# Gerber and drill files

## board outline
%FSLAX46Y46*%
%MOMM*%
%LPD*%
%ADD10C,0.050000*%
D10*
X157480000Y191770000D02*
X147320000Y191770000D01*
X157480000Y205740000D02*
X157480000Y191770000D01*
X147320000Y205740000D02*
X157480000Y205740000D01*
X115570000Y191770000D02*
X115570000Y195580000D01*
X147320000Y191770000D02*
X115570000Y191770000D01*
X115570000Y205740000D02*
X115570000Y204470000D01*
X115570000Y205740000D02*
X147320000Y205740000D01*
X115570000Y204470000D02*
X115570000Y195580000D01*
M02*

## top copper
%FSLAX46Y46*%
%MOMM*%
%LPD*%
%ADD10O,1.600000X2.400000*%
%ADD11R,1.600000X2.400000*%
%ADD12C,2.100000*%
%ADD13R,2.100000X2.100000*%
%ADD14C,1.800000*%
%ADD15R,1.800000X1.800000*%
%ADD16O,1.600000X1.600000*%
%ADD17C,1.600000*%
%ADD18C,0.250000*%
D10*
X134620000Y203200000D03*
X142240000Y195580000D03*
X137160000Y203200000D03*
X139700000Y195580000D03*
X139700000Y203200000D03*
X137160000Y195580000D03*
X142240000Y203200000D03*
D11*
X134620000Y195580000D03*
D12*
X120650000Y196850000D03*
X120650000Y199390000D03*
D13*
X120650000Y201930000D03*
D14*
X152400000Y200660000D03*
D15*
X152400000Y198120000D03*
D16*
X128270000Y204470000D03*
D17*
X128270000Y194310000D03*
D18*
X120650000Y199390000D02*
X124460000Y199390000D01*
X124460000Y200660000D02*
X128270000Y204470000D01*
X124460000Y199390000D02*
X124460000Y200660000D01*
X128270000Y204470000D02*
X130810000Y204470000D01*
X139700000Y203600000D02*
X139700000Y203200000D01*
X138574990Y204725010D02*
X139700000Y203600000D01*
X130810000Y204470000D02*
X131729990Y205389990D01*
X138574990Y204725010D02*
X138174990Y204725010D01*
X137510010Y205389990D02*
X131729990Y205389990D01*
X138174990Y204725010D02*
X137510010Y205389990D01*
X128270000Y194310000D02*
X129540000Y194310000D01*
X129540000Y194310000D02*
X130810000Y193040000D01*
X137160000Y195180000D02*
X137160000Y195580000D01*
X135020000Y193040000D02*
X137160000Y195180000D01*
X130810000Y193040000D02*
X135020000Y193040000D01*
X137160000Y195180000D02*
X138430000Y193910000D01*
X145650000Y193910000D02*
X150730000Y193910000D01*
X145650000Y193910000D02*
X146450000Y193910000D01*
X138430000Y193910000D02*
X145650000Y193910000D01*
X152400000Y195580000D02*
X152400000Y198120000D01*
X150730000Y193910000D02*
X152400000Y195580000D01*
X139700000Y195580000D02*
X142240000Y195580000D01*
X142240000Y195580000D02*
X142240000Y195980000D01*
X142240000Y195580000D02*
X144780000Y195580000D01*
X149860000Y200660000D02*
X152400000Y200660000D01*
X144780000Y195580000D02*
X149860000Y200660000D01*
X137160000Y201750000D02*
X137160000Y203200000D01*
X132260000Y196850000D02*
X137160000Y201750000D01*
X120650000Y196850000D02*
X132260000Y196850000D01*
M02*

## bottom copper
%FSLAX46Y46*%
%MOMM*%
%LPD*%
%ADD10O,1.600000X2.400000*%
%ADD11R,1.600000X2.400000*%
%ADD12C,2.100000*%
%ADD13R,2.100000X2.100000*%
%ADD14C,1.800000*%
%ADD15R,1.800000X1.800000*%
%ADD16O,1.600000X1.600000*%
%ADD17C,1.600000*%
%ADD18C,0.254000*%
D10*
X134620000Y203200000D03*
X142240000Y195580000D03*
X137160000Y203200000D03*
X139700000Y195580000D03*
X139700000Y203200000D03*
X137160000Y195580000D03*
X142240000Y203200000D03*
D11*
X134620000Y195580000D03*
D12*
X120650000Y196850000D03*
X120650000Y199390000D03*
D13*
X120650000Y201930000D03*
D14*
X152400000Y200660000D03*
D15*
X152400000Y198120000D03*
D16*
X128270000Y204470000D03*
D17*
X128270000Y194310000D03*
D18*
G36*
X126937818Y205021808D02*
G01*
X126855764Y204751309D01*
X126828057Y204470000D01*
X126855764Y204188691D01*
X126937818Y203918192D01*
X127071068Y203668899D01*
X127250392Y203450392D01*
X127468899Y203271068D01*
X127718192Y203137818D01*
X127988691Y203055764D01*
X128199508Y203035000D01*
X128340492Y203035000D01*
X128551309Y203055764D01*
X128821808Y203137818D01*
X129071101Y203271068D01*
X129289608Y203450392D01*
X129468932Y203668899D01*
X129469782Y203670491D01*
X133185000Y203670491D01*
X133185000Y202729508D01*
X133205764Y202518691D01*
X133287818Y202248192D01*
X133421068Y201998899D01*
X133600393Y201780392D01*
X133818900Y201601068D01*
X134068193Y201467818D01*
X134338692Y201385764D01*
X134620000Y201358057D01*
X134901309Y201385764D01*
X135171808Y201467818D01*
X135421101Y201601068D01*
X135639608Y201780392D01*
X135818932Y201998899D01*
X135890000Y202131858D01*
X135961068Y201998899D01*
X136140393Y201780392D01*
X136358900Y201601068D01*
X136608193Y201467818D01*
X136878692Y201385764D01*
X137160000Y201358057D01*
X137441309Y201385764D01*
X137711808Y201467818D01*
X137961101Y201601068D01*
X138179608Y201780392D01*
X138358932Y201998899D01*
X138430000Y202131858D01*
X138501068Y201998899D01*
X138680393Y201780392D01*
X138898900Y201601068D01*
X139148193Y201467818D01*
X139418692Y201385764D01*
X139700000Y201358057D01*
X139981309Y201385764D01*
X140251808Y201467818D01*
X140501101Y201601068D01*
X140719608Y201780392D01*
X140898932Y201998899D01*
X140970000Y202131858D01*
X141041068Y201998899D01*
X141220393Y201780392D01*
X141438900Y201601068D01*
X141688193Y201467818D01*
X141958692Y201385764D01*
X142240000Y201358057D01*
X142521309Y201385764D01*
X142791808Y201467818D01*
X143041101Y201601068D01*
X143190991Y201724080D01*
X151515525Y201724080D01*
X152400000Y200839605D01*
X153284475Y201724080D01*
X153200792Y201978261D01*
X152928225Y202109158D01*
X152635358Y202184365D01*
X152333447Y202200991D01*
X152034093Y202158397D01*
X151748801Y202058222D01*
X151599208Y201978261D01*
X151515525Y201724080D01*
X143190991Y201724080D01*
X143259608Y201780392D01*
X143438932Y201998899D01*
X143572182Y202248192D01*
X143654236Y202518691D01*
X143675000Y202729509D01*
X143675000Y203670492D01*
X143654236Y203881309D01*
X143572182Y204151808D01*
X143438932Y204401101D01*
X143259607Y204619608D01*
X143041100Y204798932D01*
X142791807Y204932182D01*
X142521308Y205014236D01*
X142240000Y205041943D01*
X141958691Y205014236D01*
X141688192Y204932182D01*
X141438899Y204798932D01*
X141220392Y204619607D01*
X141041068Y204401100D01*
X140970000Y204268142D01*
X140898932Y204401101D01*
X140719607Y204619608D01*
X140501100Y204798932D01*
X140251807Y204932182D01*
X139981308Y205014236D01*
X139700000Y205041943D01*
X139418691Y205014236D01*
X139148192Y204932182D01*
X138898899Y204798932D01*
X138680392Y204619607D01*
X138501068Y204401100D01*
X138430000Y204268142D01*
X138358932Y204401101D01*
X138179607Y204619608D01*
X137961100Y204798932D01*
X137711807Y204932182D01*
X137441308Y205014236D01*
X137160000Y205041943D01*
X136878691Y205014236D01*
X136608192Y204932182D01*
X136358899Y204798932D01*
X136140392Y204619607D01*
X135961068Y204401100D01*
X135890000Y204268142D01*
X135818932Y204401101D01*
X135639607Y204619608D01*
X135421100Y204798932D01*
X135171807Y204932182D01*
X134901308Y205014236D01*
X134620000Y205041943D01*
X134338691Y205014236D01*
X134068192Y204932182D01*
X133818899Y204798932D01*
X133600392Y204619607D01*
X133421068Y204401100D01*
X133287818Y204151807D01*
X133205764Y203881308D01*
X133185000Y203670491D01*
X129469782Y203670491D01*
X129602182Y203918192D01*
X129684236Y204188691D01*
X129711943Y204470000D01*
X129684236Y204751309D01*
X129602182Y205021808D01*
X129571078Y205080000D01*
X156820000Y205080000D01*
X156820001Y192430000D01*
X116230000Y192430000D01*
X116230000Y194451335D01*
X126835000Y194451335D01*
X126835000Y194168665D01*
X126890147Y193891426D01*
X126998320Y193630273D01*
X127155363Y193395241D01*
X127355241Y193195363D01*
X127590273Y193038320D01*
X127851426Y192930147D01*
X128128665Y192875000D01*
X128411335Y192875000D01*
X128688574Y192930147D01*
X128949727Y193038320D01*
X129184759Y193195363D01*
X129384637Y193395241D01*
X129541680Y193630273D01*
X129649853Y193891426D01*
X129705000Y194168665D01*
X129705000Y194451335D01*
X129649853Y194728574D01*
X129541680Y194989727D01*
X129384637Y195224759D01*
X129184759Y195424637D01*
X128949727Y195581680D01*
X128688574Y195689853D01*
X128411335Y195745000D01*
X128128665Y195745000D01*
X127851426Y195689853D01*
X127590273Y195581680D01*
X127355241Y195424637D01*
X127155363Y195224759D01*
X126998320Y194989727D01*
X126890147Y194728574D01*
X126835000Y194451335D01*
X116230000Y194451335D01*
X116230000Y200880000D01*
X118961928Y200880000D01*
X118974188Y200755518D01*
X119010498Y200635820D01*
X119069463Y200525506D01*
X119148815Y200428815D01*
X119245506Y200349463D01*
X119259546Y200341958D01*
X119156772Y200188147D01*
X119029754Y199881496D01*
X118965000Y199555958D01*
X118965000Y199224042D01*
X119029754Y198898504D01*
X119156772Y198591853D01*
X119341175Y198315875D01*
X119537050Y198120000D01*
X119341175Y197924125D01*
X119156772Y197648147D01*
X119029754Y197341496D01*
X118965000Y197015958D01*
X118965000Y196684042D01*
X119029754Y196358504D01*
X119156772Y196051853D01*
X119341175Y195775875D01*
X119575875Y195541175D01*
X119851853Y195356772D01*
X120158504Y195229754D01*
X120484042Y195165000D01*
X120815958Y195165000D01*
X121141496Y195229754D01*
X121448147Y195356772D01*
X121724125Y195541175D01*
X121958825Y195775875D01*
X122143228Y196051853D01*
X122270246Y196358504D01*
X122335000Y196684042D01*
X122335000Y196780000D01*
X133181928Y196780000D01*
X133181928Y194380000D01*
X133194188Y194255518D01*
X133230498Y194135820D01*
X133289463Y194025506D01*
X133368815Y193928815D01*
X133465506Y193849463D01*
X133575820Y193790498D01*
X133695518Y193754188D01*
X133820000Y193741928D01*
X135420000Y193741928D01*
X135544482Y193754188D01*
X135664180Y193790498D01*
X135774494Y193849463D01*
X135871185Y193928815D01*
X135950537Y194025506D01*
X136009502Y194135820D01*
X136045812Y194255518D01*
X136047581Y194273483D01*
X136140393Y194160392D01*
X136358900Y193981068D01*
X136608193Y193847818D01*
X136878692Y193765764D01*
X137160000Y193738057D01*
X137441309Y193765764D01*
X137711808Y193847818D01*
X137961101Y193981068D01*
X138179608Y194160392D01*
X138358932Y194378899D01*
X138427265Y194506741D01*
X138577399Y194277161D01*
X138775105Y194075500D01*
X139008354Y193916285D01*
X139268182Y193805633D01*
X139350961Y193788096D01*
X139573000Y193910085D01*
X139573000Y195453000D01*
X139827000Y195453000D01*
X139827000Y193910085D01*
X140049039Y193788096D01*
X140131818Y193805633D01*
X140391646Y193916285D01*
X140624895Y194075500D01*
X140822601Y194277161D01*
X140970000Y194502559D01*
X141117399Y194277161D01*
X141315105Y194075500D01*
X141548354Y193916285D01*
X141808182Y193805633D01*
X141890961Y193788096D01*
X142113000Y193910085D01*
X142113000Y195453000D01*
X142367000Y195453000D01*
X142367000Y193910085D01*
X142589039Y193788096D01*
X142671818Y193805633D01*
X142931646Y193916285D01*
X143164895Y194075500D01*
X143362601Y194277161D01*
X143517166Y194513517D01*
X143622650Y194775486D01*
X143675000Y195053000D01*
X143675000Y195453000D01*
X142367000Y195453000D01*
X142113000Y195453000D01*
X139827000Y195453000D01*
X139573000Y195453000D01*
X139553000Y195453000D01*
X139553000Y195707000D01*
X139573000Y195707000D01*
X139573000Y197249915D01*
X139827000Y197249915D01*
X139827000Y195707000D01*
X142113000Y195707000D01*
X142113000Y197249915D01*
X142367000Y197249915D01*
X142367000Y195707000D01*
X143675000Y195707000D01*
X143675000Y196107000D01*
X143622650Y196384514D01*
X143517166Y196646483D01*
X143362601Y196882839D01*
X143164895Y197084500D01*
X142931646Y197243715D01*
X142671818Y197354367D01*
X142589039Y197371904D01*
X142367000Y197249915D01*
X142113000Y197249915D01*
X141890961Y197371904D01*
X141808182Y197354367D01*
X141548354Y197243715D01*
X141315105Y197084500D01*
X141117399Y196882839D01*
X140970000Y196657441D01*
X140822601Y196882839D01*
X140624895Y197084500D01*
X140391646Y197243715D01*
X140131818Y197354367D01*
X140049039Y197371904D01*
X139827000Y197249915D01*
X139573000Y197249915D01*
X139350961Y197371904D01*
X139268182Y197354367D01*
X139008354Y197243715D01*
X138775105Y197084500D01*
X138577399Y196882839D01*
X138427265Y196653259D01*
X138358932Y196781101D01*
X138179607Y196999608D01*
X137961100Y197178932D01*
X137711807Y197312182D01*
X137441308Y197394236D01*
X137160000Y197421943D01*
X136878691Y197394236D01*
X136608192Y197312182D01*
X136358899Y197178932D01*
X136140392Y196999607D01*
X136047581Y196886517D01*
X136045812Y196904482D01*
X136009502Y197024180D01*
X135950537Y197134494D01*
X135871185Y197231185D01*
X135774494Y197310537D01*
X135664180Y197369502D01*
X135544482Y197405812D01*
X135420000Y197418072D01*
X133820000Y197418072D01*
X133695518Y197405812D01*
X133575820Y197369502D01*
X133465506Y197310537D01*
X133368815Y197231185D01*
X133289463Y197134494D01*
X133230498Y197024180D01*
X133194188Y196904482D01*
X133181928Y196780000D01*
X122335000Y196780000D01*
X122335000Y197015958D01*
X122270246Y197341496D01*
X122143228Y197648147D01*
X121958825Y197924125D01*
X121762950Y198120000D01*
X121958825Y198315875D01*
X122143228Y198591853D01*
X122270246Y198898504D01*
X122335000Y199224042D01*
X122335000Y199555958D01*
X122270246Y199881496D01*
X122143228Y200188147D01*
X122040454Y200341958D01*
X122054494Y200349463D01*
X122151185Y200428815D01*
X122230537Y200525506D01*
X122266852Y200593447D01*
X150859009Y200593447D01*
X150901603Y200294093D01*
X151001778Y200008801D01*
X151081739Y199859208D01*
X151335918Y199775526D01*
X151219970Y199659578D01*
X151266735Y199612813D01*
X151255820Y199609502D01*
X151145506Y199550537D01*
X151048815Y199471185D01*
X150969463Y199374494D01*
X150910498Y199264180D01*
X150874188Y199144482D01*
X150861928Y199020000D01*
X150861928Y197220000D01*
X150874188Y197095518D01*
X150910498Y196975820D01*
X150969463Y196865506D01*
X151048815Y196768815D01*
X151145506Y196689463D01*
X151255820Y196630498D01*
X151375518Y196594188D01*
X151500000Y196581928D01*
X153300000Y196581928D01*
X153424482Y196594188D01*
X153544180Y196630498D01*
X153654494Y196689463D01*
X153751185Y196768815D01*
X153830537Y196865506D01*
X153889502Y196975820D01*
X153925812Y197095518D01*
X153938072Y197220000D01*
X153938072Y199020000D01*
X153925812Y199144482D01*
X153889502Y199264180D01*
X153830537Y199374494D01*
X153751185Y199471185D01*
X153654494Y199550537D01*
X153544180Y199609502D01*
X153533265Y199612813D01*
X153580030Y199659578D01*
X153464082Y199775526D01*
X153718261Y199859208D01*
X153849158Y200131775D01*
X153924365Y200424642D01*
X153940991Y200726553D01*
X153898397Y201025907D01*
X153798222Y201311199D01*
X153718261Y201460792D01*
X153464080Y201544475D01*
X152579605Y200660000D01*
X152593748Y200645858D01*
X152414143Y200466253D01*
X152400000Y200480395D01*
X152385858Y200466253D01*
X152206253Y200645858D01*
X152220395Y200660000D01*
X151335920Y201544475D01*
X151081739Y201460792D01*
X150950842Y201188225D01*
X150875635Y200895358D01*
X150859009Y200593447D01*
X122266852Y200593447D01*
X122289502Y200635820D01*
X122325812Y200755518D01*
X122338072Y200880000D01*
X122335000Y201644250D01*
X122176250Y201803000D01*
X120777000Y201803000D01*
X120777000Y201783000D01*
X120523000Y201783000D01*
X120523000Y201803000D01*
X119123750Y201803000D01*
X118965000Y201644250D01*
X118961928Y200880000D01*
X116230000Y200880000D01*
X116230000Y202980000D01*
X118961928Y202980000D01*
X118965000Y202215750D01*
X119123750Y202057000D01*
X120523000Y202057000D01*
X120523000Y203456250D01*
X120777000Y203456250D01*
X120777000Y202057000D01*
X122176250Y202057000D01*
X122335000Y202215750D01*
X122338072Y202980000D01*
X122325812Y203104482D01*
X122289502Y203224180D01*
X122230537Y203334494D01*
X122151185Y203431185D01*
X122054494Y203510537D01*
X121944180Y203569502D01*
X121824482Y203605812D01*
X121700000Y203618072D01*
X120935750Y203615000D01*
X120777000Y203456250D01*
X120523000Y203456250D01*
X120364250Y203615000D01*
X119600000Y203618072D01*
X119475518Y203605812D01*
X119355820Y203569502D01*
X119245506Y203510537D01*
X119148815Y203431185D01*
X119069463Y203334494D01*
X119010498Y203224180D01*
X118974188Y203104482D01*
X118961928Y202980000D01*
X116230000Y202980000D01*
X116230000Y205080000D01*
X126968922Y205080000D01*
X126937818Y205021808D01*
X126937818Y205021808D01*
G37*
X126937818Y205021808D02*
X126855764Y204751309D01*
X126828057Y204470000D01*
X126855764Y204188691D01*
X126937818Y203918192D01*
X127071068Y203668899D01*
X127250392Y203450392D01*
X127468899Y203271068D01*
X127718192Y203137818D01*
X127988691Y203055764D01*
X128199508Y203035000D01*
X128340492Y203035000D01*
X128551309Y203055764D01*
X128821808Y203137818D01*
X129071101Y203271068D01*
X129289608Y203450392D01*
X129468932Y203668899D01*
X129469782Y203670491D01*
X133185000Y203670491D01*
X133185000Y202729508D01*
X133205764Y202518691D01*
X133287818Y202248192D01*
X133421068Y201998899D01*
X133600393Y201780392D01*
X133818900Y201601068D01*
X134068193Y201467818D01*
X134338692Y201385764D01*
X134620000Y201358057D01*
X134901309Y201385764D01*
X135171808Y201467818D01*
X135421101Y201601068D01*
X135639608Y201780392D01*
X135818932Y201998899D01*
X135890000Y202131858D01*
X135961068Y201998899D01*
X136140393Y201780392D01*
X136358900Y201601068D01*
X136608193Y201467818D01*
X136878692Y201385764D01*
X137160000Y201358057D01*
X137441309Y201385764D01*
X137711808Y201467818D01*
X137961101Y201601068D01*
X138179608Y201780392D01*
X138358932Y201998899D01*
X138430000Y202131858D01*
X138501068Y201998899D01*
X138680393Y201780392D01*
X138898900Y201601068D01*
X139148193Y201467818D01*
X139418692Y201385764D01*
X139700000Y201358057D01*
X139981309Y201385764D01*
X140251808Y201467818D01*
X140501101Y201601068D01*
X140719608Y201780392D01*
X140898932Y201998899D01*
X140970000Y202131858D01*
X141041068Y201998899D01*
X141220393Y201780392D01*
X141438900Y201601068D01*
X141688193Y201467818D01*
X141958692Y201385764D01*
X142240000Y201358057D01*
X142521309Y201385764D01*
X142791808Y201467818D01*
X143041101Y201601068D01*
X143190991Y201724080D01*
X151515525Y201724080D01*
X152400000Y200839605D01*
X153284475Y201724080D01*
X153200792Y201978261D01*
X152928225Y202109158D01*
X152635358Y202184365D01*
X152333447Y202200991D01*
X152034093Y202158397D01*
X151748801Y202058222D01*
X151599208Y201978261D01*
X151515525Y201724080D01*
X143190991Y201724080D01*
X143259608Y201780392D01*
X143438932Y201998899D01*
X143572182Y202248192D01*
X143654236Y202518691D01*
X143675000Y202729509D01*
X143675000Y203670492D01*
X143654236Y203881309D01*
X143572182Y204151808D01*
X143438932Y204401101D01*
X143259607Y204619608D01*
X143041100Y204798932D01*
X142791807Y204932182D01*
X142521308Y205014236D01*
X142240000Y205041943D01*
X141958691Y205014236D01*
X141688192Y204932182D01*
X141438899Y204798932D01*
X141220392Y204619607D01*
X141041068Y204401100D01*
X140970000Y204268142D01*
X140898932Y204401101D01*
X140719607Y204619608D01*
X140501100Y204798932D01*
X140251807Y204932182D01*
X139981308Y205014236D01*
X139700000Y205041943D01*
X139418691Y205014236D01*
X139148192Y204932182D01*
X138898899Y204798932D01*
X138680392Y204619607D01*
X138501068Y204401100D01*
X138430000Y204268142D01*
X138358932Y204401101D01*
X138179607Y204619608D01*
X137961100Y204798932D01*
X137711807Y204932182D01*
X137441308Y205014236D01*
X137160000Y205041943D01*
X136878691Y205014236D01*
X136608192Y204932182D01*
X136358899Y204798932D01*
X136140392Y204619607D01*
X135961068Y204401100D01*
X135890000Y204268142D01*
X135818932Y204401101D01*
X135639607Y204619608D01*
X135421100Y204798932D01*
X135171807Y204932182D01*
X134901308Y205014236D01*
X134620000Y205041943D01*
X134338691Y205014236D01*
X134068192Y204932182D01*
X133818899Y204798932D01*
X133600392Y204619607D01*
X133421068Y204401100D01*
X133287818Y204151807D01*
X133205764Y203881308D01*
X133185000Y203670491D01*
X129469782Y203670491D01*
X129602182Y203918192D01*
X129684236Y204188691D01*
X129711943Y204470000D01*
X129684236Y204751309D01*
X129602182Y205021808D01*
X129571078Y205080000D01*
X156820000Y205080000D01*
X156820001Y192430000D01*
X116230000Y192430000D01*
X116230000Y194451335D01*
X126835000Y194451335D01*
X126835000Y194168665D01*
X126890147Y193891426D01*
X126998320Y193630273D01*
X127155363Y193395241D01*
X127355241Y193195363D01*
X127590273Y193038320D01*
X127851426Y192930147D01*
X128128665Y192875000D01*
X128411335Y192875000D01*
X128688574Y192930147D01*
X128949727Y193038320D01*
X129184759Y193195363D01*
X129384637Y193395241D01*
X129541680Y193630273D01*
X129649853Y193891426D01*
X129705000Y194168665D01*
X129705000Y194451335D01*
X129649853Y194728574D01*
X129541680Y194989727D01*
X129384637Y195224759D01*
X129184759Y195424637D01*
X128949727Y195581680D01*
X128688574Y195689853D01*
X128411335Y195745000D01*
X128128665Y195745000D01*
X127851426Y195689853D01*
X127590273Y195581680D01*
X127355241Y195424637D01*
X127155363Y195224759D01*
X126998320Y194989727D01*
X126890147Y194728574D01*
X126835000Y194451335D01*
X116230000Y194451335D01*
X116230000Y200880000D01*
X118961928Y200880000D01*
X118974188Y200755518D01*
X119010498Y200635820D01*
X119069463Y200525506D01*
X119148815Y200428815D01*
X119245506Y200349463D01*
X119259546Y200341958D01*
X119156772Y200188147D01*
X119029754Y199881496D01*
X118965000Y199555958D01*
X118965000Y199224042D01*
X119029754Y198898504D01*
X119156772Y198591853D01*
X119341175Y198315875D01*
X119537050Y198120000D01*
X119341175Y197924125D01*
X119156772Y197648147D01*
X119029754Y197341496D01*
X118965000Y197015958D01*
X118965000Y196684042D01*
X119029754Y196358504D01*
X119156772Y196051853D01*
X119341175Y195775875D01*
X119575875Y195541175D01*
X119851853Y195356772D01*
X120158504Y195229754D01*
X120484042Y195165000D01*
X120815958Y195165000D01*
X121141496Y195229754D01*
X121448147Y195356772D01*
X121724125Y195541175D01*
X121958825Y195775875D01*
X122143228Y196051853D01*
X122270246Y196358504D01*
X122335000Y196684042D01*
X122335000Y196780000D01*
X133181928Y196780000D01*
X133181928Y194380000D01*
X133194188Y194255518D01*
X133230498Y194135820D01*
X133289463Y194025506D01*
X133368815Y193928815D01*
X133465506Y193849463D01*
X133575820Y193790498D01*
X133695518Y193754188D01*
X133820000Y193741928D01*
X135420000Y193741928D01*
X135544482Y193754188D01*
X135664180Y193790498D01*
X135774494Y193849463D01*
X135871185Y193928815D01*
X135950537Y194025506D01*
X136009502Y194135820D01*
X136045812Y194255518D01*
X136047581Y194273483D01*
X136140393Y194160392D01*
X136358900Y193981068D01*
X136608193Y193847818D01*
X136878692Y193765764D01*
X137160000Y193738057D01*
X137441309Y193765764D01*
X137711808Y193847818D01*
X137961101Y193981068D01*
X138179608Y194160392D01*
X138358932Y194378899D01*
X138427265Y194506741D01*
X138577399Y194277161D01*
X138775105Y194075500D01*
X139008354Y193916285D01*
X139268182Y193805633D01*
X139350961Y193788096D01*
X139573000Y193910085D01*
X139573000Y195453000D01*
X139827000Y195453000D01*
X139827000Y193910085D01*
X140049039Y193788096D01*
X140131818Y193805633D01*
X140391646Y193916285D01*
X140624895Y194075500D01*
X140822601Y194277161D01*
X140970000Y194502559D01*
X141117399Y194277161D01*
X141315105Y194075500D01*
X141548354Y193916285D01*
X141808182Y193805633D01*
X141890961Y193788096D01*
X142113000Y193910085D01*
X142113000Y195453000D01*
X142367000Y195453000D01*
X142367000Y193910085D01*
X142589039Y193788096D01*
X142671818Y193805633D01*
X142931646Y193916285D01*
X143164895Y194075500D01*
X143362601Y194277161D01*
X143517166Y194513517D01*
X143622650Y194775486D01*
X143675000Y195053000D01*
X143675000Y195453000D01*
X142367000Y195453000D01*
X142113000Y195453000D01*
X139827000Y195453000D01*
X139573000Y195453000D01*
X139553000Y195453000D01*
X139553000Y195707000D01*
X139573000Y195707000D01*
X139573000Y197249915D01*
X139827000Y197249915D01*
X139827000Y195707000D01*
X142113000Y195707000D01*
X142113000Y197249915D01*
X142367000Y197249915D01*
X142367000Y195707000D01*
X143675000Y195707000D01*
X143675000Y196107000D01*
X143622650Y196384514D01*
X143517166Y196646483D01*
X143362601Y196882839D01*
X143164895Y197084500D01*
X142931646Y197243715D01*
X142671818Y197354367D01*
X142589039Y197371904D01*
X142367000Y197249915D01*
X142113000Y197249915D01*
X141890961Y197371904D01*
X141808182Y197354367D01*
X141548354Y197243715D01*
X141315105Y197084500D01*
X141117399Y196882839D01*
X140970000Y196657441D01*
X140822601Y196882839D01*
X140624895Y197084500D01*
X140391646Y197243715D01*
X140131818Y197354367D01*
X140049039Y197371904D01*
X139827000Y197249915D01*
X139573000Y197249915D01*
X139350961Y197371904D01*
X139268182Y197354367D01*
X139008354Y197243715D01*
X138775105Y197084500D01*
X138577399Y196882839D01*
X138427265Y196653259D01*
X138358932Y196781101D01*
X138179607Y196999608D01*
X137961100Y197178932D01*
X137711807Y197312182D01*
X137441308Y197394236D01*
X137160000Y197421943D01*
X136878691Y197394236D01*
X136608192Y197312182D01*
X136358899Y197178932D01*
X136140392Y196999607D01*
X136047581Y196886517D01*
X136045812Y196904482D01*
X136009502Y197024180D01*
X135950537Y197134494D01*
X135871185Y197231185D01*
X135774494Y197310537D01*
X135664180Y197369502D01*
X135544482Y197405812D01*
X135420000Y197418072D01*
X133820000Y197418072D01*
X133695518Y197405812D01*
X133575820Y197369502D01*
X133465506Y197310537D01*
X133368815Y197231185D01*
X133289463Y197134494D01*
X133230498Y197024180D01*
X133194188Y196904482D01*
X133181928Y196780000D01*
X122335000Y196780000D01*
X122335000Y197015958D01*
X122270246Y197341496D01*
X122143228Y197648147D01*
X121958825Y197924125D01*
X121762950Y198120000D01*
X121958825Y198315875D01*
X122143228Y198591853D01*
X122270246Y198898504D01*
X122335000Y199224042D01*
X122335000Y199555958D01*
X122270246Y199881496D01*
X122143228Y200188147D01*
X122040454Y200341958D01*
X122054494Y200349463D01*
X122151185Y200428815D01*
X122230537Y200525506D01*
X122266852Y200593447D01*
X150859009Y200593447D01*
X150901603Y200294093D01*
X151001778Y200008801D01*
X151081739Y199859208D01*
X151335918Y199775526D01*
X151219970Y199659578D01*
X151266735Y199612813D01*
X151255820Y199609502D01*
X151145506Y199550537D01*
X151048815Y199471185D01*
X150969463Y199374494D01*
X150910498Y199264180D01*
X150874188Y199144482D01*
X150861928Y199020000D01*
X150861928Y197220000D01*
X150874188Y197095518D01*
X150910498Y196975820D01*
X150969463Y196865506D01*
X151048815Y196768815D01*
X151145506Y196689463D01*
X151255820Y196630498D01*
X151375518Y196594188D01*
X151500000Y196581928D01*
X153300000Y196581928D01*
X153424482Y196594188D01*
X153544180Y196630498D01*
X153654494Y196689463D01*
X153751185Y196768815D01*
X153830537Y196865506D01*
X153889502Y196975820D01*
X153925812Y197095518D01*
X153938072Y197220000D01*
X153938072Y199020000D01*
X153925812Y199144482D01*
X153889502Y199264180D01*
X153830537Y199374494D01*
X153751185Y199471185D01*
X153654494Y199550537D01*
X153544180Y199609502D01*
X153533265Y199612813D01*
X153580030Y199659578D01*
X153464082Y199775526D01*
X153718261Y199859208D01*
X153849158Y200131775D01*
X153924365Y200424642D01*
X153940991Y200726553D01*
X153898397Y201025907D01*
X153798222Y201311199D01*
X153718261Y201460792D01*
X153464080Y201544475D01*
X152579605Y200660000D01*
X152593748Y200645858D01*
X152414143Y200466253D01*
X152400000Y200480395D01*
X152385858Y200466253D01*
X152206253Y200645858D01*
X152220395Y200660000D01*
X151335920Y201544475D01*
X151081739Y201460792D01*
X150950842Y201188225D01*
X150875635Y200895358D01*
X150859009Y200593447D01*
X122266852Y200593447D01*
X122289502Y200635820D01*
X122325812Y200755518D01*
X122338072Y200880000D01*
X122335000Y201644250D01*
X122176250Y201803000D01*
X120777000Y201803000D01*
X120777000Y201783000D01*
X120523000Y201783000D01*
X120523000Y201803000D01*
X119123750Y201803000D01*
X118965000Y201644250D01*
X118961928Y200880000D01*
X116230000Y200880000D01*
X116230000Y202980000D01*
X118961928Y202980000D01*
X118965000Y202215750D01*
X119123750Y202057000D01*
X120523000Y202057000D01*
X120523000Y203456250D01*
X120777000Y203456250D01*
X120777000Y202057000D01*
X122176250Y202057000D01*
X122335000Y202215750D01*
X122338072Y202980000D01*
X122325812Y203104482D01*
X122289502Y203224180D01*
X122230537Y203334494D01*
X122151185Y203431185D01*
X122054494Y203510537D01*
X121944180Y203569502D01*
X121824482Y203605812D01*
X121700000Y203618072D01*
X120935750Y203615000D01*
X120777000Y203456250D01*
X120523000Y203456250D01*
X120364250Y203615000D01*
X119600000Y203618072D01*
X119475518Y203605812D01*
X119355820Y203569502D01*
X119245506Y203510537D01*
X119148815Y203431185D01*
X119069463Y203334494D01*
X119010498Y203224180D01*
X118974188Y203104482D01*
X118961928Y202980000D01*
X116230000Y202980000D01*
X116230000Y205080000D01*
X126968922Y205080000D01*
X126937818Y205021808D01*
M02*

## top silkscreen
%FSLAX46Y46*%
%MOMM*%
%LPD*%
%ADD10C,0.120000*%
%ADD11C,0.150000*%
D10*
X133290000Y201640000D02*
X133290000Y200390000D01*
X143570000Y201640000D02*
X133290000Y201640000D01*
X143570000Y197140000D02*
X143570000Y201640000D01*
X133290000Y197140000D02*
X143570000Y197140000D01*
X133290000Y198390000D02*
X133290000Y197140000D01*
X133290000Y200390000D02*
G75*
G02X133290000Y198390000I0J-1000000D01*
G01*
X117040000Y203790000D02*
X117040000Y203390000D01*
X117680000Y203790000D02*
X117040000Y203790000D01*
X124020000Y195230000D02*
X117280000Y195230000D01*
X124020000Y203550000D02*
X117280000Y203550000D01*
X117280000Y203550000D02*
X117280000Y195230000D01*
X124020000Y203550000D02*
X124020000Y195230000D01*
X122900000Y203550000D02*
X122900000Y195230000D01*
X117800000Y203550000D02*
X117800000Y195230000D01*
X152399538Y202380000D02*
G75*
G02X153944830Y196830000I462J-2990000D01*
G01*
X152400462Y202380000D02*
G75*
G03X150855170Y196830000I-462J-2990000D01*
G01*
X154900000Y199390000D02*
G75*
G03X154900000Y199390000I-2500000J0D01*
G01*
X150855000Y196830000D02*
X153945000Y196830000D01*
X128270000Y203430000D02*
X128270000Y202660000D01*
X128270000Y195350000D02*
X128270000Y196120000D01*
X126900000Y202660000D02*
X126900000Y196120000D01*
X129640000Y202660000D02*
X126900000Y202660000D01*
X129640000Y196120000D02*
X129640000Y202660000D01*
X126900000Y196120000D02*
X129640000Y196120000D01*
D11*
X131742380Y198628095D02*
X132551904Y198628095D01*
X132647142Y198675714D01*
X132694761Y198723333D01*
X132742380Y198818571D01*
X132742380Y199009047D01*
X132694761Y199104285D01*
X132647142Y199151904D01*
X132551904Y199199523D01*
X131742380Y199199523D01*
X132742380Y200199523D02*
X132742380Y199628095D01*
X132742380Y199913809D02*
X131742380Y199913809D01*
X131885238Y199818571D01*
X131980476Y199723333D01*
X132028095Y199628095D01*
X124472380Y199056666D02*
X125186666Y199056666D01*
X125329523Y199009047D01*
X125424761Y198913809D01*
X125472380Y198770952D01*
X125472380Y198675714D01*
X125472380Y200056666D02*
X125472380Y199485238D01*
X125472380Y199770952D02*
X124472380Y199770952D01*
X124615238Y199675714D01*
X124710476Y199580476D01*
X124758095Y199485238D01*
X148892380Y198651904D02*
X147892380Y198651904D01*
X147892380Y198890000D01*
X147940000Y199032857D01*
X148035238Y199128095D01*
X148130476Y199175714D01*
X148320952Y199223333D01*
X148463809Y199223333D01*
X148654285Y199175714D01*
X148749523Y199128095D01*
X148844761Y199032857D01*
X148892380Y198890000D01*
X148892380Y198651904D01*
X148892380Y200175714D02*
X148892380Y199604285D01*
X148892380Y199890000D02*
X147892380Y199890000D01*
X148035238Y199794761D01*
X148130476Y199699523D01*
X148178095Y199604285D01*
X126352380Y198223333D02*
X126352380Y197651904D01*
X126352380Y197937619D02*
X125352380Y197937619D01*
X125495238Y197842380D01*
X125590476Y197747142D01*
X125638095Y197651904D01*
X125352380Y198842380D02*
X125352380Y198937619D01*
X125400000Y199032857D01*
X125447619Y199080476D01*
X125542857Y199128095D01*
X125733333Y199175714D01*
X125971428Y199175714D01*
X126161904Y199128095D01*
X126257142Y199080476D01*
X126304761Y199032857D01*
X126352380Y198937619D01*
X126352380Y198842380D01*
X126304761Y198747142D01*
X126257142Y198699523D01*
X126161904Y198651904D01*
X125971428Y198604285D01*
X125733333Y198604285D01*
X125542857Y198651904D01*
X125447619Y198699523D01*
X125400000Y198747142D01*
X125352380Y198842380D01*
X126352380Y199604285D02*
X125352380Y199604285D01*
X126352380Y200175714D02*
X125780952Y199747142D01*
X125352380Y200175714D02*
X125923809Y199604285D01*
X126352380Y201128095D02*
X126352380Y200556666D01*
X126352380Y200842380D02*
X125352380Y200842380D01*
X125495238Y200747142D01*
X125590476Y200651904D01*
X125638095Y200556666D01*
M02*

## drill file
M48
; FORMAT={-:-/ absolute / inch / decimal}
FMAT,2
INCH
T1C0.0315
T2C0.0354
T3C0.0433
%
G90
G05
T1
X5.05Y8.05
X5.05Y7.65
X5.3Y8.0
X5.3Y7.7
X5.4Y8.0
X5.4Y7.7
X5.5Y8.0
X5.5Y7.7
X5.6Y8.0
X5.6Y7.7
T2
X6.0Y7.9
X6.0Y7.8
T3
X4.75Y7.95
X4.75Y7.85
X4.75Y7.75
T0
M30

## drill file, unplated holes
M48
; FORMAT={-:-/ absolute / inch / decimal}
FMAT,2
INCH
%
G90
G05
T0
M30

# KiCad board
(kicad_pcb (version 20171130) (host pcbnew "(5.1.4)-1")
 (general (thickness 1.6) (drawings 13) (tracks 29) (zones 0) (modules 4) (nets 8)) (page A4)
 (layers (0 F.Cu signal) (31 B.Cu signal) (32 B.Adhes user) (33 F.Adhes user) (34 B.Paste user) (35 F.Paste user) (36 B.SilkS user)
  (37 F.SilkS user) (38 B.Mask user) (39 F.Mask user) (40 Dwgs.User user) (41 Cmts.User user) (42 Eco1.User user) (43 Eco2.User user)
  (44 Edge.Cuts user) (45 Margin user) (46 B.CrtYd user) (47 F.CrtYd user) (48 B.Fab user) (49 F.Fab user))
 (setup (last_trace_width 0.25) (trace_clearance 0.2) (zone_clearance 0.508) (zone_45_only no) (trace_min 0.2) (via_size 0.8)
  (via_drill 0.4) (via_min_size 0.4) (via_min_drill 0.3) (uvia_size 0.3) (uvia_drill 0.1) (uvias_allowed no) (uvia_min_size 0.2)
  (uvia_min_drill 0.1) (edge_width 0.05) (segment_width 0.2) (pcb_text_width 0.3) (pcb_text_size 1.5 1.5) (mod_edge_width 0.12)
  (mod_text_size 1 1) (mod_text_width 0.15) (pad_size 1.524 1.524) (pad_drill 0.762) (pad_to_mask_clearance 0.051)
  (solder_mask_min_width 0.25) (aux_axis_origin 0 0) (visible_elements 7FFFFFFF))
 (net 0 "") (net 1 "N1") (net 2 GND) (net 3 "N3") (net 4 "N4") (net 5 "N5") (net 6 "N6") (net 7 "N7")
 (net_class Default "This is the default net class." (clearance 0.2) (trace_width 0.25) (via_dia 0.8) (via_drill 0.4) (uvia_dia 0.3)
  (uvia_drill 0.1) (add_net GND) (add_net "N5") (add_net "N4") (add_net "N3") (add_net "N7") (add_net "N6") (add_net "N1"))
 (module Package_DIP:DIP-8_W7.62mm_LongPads (layer F.Cu) (at 134.62 -195.58 90)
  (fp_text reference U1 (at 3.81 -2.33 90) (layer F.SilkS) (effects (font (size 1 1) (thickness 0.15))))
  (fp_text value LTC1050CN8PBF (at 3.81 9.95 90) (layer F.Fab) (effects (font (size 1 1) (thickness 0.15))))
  (fp_line (start 6.06 -1.33) (end 4.81 -1.33) (layer F.SilkS) (width 0.12))
  (fp_line (start 6.06 8.95) (end 6.06 -1.33) (layer F.SilkS) (width 0.12))
  (fp_line (start 1.56 8.95) (end 6.06 8.95) (layer F.SilkS) (width 0.12))
  (fp_line (start 1.56 -1.33) (end 1.56 8.95) (layer F.SilkS) (width 0.12))
  (fp_line (start 2.81 -1.33) (end 1.56 -1.33) (layer F.SilkS) (width 0.12))
  (fp_arc (start 3.81 -1.33) (end 2.81 -1.33) (angle -180) (layer F.SilkS) (width 0.12))
  (pad 8 thru_hole oval (at 7.62 0 90) (size 2.4 1.6) (drill 0.8) (layers *.Cu *.Mask) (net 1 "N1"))
  (pad 4 thru_hole oval (at 0 7.62 90) (size 2.4 1.6) (drill 0.8) (layers *.Cu *.Mask) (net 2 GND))
  (pad 7 thru_hole oval (at 7.62 2.54 90) (size 2.4 1.6) (drill 0.8) (layers *.Cu *.Mask) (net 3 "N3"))
  (pad 3 thru_hole oval (at 0 5.08 90) (size 2.4 1.6) (drill 0.8) (layers *.Cu *.Mask) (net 2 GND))
  (pad 6 thru_hole oval (at 7.62 5.08 90) (size 2.4 1.6) (drill 0.8) (layers *.Cu *.Mask) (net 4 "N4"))
  (pad 2 thru_hole oval (at 0 2.54 90) (size 2.4 1.6) (drill 0.8) (layers *.Cu *.Mask) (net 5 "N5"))
  (pad 5 thru_hole oval (at 7.62 7.62 90) (size 2.4 1.6) (drill 0.8) (layers *.Cu *.Mask) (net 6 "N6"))
  (pad 1 thru_hole rect (at 0 0 90) (size 2.4 1.6) (drill 0.8) (layers *.Cu *.Mask) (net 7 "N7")))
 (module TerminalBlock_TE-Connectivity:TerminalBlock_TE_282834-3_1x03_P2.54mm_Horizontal (layer F.Cu) (at 120.65 -201.93 270)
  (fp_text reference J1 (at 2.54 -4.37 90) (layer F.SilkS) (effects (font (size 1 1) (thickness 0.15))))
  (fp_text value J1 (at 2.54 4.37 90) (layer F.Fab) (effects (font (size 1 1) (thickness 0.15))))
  (fp_line (start -1.86 3.61) (end -1.46 3.61) (layer F.SilkS) (width 0.12))
  (fp_line (start -1.86 2.97) (end -1.86 3.61) (layer F.SilkS) (width 0.12))
  (fp_line (start 6.7 -3.37) (end 6.7 3.37) (layer F.SilkS) (width 0.12))
  (fp_line (start -1.62 -3.37) (end -1.62 3.37) (layer F.SilkS) (width 0.12))
  (fp_line (start -1.62 3.37) (end 6.7 3.37) (layer F.SilkS) (width 0.12))
  (fp_line (start -1.62 -3.37) (end 6.7 -3.37) (layer F.SilkS) (width 0.12))
  (fp_line (start -1.62 -2.25) (end 6.7 -2.25) (layer F.SilkS) (width 0.12))
  (fp_line (start -1.62 2.85) (end 6.7 2.85) (layer F.SilkS) (width 0.12))
  (pad 3 thru_hole circle (at 5.08 0 270) (size 2.1 2.1) (drill 1.1) (layers *.Cu *.Mask) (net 3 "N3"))
  (pad 2 thru_hole circle (at 2.54 0 270) (size 2.1 2.1) (drill 1.1) (layers *.Cu *.Mask) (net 4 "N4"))
  (pad 1 thru_hole rect (at 0 0 270) (size 2.1 2.1) (drill 1.1) (layers *.Cu *.Mask) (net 2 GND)))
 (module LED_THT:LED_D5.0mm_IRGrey (layer F.Cu) (at 152.4 -198.12 90)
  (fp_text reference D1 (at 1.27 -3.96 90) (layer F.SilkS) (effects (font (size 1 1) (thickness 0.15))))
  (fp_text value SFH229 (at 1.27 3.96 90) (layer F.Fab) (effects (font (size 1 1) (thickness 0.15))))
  (fp_arc (start 1.27 0) (end -1.29 1.54483) (angle -148.9) (layer F.SilkS) (width 0.12))
  (fp_arc (start 1.27 0) (end -1.29 -1.54483) (angle 148.9) (layer F.SilkS) (width 0.12))
  (fp_circle (center 1.27 0) (end 3.77 0) (layer F.SilkS) (width 0.12))
  (fp_line (start -1.29 -1.545) (end -1.29 1.545) (layer F.SilkS) (width 0.12))
  (pad 2 thru_hole circle (at 2.54 0 90) (size 1.8 1.8) (drill 0.9) (layers *.Cu *.Mask) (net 2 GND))
  (pad 1 thru_hole rect (at 0 0 90) (size 1.8 1.8) (drill 0.9) (layers *.Cu *.Mask) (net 5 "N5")))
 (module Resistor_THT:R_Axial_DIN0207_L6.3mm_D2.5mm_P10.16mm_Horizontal (layer F.Cu) (at 128.27 -194.31 90)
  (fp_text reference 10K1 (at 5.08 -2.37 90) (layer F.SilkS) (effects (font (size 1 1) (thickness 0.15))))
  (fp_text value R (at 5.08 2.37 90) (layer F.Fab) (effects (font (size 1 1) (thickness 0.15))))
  (fp_line (start 9.12 0) (end 8.35 0) (layer F.SilkS) (width 0.12))
  (fp_line (start 1.04 0) (end 1.81 0) (layer F.SilkS) (width 0.12))
  (fp_line (start 8.35 -1.37) (end 1.81 -1.37) (layer F.SilkS) (width 0.12))
  (fp_line (start 8.35 1.37) (end 8.35 -1.37) (layer F.SilkS) (width 0.12))
  (fp_line (start 1.81 1.37) (end 8.35 1.37) (layer F.SilkS) (width 0.12))
  (fp_line (start 1.81 -1.37) (end 1.81 1.37) (layer F.SilkS) (width 0.12))
  (pad 2 thru_hole oval (at 10.16 0 90) (size 1.6 1.6) (drill 0.8) (layers *.Cu *.Mask) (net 4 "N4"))
  (pad 1 thru_hole circle (at 0 0 90) (size 1.6 1.6) (drill 0.8) (layers *.Cu *.Mask) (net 5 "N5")))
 (gr_line (start 157.48 -191.77) (end 147.32 -191.77) (layer Edge.Cuts) (width 0.05))
 (gr_line (start 157.48 -205.74) (end 157.48 -191.77) (layer Edge.Cuts) (width 0.05))
 (gr_line (start 147.32 -205.74) (end 157.48 -205.74) (layer Edge.Cuts) (width 0.05))
 (gr_line (start 115.57 -191.77) (end 115.57 -195.58) (layer Edge.Cuts) (width 0.05))
 (gr_line (start 147.32 -191.77) (end 115.57 -191.77) (layer Edge.Cuts) (width 0.05))
 (gr_line (start 115.57 -205.74) (end 115.57 -204.47) (layer Edge.Cuts) (width 0.05))
 (gr_line (start 115.57 -205.74) (end 147.32 -205.74) (layer Edge.Cuts) (width 0.05))
 (gr_line (start 115.57 -204.47) (end 115.57 -195.58) (layer Edge.Cuts) (width 0.05))
 (segment (start 120.65 -199.39) (end 124.46 -199.39) (width 0.25) (layer F.Cu) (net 4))
 (segment (start 124.46 -200.66) (end 128.27 -204.47) (width 0.25) (layer F.Cu) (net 4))
 (segment (start 124.46 -199.39) (end 124.46 -200.66) (width 0.25) (layer F.Cu) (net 4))
 (segment (start 128.27 -204.47) (end 130.81 -204.47) (width 0.25) (layer F.Cu) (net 4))
 (segment (start 139.7 -203.6) (end 139.7 -203.2) (width 0.25) (layer F.Cu) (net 4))
 (segment (start 138.57499 -204.72501) (end 139.7 -203.6) (width 0.25) (layer F.Cu) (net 4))
 (segment (start 130.81 -204.47) (end 131.72999 -205.38999) (width 0.25) (layer F.Cu) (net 4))
 (segment (start 138.57499 -204.72501) (end 138.17499 -204.72501) (width 0.25) (layer F.Cu) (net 4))
 (segment (start 137.51001 -205.38999) (end 131.72999 -205.38999) (width 0.25) (layer F.Cu) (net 4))
 (segment (start 138.17499 -204.72501) (end 137.51001 -205.38999) (width 0.25) (layer F.Cu) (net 4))
 (segment (start 128.27 -194.31) (end 129.54 -194.31) (width 0.25) (layer F.Cu) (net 5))
 (segment (start 129.54 -194.31) (end 130.81 -193.04) (width 0.25) (layer F.Cu) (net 5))
 (segment (start 137.16 -195.18) (end 137.16 -195.58) (width 0.25) (layer F.Cu) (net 5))
 (segment (start 135.02 -193.04) (end 137.16 -195.18) (width 0.25) (layer F.Cu) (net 5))
 (segment (start 130.81 -193.04) (end 135.02 -193.04) (width 0.25) (layer F.Cu) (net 5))
 (segment (start 137.16 -195.18) (end 138.43 -193.91) (width 0.25) (layer F.Cu) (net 5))
 (segment (start 145.65 -193.91) (end 150.73 -193.91) (width 0.25) (layer F.Cu) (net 5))
 (segment (start 145.65 -193.91) (end 146.45 -193.91) (width 0.25) (layer F.Cu) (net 5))
 (segment (start 138.43 -193.91) (end 145.65 -193.91) (width 0.25) (layer F.Cu) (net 5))
 (segment (start 152.4 -195.58) (end 152.4 -198.12) (width 0.25) (layer F.Cu) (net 5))
 (segment (start 150.73 -193.91) (end 152.4 -195.58) (width 0.25) (layer F.Cu) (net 5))
 (segment (start 139.7 -195.58) (end 142.24 -195.58) (width 0.25) (layer F.Cu) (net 2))
 (segment (start 142.24 -195.58) (end 142.24 -195.98) (width 0.25) (layer F.Cu) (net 2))
 (segment (start 142.24 -195.58) (end 144.78 -195.58) (width 0.25) (layer F.Cu) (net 2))
 (segment (start 149.86 -200.66) (end 152.4 -200.66) (width 0.25) (layer F.Cu) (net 2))
 (segment (start 144.78 -195.58) (end 149.86 -200.66) (width 0.25) (layer F.Cu) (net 2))
 (segment (start 137.16 -201.75) (end 137.16 -203.2) (width 0.25) (layer F.Cu) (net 3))
 (segment (start 132.26 -196.85) (end 137.16 -201.75) (width 0.25) (layer F.Cu) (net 3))
 (segment (start 120.65 -196.85) (end 132.26 -196.85) (width 0.25) (layer F.Cu) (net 3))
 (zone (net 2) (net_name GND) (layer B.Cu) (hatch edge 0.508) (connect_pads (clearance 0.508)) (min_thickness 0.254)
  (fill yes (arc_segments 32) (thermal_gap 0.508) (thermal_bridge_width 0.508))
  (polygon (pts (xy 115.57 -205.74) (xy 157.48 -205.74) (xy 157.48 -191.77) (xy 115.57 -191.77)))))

